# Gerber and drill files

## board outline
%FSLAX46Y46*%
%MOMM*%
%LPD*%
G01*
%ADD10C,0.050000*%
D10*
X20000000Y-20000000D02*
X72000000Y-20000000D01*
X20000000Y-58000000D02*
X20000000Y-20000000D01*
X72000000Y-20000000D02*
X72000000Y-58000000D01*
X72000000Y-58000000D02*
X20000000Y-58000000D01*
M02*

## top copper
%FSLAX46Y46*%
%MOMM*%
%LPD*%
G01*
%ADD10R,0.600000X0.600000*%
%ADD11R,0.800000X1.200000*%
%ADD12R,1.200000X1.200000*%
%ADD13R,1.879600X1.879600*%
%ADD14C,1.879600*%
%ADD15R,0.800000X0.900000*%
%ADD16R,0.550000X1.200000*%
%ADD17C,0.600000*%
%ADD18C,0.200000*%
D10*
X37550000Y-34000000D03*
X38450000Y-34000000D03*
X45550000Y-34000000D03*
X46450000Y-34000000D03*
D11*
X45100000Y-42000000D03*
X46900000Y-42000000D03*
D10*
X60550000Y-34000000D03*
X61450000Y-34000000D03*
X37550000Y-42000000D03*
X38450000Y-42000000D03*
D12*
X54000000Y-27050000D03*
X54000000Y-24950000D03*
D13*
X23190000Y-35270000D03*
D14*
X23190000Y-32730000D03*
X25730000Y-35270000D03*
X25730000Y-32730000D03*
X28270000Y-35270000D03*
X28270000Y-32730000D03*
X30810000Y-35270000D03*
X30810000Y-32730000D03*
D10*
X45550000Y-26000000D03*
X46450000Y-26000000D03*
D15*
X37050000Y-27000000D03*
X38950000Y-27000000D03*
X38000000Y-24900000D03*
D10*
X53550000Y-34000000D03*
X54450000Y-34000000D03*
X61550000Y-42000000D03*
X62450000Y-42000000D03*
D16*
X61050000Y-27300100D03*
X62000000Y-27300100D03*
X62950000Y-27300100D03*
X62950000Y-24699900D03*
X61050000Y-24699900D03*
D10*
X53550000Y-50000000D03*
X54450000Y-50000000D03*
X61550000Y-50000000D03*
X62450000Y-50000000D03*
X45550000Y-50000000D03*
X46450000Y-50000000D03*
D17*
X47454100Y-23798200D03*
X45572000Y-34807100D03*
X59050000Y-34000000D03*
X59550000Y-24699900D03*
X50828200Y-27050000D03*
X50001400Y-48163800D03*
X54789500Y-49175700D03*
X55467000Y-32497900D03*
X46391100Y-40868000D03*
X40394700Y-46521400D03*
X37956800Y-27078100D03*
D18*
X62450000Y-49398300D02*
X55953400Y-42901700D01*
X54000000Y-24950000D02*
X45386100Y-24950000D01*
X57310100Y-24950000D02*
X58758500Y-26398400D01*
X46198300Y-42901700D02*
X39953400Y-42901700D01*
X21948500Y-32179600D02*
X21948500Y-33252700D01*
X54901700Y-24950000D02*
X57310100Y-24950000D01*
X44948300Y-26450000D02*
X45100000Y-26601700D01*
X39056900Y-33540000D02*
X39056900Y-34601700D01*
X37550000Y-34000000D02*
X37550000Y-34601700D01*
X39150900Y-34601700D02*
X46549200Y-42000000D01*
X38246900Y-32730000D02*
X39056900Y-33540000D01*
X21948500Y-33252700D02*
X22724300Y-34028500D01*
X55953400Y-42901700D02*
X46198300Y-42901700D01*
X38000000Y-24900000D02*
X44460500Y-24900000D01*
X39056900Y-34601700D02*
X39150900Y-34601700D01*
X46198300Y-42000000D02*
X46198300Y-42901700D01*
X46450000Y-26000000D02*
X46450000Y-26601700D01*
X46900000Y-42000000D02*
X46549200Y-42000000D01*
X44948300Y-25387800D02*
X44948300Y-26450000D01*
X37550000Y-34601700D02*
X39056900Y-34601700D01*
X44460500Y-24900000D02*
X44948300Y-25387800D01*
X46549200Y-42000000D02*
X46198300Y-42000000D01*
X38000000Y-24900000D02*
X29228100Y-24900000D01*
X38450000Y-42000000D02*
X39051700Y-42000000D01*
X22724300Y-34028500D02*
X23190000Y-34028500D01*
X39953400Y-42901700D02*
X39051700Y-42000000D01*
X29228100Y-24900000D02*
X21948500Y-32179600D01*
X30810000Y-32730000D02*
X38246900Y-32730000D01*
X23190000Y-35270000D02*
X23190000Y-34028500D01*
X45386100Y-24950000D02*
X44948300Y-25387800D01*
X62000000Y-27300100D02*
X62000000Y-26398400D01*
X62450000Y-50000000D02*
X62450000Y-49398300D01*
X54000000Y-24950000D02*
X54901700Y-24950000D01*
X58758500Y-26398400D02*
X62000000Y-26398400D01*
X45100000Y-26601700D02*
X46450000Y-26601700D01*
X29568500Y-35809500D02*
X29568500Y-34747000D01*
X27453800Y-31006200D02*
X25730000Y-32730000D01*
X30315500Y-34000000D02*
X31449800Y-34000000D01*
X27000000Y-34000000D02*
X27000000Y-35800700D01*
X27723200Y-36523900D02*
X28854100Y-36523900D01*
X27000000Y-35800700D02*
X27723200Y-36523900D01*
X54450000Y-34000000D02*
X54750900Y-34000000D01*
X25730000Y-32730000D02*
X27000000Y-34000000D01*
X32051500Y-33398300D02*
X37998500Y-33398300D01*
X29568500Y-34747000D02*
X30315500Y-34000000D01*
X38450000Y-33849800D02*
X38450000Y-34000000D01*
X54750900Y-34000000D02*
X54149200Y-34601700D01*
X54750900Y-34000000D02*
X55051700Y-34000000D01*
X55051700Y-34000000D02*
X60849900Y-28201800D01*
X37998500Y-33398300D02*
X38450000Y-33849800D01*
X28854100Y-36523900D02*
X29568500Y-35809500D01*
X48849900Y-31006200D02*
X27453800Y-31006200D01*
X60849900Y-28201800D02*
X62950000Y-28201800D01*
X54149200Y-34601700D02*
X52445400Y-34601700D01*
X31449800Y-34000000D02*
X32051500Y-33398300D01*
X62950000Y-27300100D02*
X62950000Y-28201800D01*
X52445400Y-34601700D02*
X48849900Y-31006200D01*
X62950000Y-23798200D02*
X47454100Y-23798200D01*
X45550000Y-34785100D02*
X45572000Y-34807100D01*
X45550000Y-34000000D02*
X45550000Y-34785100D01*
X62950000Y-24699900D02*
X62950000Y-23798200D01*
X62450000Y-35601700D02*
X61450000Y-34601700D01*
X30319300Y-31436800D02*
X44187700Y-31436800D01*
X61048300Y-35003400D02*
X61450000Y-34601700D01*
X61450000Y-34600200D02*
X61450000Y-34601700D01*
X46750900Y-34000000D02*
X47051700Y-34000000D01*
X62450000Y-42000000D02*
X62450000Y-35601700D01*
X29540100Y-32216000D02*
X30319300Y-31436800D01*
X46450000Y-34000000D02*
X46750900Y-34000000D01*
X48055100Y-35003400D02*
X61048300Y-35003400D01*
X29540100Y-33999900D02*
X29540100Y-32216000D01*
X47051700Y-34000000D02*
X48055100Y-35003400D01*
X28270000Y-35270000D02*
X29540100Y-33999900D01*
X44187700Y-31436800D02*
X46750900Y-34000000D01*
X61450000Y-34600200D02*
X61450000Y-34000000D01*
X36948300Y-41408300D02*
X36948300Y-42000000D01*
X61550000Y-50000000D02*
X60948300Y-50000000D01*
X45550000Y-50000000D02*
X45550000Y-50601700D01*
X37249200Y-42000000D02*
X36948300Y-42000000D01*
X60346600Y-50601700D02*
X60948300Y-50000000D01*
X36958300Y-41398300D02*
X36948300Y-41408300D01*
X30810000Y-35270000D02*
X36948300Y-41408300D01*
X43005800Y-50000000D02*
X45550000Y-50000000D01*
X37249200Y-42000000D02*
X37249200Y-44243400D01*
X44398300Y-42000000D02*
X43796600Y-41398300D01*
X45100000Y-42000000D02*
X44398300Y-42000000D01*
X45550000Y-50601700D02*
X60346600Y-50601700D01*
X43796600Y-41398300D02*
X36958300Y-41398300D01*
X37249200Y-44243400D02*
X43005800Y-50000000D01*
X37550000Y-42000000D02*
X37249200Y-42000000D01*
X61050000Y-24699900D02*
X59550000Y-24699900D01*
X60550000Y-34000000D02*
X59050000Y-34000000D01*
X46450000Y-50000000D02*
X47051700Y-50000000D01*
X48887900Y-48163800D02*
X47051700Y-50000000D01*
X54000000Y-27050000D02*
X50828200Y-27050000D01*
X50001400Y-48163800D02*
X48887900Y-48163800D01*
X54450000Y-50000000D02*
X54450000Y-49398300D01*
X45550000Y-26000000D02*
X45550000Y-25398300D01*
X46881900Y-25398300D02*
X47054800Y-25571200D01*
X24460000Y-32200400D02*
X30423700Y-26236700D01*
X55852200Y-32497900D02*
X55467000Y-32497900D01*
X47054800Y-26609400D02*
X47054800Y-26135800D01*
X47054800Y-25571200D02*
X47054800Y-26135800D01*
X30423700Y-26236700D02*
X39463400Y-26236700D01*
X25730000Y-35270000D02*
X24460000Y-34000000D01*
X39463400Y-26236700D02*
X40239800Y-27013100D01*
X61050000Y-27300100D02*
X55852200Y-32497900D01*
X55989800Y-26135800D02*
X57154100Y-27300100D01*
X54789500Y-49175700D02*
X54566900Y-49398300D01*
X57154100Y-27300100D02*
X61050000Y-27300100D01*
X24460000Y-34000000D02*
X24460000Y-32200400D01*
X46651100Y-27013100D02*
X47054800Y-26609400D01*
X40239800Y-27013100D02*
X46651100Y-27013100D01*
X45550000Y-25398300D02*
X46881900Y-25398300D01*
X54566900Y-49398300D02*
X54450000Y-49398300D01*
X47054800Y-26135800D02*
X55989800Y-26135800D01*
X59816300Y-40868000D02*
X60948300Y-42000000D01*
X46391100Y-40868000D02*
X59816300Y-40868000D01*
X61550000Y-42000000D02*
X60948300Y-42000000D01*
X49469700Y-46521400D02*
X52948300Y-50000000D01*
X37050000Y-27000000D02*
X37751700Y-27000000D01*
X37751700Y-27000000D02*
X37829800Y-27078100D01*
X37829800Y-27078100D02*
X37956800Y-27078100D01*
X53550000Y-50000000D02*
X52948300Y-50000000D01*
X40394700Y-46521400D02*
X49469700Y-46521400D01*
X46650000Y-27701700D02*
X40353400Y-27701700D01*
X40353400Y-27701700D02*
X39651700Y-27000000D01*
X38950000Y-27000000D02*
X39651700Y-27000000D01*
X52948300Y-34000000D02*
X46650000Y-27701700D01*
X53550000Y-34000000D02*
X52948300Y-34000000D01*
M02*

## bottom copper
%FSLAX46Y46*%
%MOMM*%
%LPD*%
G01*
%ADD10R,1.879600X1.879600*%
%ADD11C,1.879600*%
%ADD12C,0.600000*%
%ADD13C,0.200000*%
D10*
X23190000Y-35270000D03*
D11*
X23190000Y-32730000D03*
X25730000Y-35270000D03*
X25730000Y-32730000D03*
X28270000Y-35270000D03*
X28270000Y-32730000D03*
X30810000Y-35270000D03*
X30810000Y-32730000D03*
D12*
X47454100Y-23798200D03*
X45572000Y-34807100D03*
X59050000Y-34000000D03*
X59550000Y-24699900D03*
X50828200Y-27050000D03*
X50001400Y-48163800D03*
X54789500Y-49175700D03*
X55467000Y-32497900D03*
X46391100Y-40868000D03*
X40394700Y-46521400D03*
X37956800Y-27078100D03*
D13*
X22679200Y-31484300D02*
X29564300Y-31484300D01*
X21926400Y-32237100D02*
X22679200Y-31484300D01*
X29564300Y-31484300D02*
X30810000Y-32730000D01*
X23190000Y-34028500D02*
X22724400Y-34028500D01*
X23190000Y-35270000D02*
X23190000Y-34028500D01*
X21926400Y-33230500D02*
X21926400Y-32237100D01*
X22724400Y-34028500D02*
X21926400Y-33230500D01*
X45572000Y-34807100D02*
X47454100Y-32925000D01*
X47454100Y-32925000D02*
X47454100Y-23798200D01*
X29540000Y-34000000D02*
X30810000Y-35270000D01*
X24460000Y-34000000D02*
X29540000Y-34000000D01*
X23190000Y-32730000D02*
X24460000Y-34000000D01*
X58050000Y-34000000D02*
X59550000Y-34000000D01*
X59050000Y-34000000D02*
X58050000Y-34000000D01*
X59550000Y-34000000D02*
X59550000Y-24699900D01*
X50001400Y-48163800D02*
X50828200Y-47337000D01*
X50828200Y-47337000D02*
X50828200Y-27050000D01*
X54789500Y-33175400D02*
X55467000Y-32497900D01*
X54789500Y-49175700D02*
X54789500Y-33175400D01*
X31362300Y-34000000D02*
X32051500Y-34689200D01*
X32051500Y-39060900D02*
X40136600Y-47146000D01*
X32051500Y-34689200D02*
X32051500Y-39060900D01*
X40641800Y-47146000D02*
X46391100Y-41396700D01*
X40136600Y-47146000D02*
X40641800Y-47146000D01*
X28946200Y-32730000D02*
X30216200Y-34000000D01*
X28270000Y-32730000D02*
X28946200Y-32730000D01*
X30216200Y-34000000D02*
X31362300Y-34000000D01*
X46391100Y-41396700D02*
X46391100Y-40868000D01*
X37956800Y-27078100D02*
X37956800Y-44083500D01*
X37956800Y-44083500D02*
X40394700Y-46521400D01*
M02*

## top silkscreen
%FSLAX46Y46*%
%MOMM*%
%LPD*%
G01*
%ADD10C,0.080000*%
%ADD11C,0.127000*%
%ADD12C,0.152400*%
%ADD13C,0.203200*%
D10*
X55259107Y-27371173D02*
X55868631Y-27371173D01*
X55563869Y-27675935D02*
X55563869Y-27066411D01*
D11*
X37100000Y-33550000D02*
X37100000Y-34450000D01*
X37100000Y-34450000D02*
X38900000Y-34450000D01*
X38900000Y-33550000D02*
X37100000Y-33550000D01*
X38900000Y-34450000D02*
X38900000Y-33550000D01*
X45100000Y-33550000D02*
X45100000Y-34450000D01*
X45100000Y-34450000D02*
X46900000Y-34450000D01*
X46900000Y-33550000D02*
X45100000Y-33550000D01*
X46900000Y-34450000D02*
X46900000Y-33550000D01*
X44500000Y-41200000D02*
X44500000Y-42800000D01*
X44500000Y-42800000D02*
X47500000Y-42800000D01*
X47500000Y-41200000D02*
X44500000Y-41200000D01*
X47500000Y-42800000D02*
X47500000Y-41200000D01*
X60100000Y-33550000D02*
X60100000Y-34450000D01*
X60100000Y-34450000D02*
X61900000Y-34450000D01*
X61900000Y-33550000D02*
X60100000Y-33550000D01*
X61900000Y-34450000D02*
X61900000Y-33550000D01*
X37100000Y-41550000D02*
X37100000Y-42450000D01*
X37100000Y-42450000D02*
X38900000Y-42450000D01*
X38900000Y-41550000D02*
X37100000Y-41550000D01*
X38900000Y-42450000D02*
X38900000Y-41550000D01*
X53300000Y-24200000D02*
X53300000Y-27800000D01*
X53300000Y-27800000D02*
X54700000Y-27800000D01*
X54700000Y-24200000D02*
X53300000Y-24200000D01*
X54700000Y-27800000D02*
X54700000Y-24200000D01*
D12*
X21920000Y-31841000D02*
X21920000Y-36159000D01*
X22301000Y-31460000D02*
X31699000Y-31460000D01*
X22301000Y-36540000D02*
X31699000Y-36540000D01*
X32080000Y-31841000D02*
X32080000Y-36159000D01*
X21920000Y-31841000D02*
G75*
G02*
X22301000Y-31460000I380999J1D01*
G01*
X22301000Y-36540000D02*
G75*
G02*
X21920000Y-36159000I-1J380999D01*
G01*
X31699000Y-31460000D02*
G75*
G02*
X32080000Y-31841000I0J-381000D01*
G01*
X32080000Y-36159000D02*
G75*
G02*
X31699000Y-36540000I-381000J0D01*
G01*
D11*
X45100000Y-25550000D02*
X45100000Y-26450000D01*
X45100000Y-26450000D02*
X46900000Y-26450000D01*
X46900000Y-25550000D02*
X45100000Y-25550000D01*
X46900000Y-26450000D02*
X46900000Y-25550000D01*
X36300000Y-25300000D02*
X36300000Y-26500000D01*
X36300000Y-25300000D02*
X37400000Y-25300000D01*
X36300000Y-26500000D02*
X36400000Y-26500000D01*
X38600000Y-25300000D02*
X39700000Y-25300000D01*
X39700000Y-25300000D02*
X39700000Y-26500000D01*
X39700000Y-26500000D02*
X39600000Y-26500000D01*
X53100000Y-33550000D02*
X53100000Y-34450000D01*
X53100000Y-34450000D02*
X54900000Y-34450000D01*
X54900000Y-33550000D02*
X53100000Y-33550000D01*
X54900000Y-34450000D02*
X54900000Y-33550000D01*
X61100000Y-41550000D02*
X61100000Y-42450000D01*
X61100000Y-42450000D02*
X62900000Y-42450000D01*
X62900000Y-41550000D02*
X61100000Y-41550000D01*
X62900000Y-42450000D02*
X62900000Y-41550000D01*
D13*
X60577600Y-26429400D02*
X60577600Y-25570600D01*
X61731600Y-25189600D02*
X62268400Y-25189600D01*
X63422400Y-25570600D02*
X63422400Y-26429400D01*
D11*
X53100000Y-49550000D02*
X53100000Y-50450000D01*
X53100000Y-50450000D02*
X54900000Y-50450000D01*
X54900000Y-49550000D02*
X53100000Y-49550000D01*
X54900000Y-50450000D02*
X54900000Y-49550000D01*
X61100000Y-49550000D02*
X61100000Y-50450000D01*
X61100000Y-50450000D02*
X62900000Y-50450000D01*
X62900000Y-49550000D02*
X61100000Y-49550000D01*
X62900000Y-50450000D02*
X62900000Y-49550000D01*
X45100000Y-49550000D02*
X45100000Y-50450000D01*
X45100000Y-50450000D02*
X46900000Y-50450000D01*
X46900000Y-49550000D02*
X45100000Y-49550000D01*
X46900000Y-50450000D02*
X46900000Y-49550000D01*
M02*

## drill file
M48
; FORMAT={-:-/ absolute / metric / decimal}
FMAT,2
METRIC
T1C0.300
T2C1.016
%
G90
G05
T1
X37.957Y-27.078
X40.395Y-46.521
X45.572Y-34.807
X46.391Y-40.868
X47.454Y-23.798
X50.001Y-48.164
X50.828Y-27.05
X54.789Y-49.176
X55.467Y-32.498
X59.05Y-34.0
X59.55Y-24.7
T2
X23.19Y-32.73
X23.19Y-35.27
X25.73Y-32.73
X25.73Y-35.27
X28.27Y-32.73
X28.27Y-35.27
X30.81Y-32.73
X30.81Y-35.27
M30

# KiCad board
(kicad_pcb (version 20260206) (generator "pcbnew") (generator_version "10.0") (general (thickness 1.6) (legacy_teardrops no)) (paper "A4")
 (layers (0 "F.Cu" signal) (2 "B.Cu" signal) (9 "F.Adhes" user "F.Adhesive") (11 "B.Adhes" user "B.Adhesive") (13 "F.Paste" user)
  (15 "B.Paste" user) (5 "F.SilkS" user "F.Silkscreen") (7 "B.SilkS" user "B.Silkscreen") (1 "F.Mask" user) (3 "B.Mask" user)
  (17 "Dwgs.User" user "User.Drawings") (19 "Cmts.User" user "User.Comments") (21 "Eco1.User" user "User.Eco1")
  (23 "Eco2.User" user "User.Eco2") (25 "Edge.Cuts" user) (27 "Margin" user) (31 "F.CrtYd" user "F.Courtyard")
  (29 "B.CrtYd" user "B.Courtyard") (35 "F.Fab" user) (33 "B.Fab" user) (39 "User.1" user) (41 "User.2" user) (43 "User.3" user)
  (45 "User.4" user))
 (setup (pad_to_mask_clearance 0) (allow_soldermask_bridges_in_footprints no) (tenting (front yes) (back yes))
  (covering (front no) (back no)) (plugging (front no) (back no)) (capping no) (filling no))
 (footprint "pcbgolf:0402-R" (layer "F.Cu") (at 38 34)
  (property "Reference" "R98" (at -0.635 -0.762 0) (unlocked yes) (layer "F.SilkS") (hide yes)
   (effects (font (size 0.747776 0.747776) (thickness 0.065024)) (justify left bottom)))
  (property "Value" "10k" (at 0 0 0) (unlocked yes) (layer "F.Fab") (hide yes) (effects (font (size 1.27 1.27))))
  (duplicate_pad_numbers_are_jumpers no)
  (fp_line (start -0.9 -0.45) (end -0.9 0.45) (stroke (width 0.127) (type solid)) (layer "F.SilkS"))
  (fp_line (start -0.9 0.45) (end 0.9 0.45) (stroke (width 0.127) (type solid)) (layer "F.SilkS"))
  (fp_line (start 0.9 -0.45) (end -0.9 -0.45) (stroke (width 0.127) (type solid)) (layer "F.SilkS"))
  (fp_line (start 0.9 0.45) (end 0.9 -0.45) (stroke (width 0.127) (type solid)) (layer "F.SilkS"))
  (pad "1" smd rect (at -0.45 0) (size 0.6 0.6) (layers "F.Cu" "F.Mask" "F.Paste") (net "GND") (solder_mask_margin 0.0508)
   (solder_paste_margin 0) (thermal_bridge_angle 0))
  (pad "2" smd rect (at 0.45 0) (size 0.6 0.6) (layers "F.Cu" "F.Mask" "F.Paste") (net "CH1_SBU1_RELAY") (solder_mask_margin 0.0508)
   (solder_paste_margin 0) (thermal_bridge_angle 0)))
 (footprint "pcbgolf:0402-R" (layer "F.Cu") (at 46 34)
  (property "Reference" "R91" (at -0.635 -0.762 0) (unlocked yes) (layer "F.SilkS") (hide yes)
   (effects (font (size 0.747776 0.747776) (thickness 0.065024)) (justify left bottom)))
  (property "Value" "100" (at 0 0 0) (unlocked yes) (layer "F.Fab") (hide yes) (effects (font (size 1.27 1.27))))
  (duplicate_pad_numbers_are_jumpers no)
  (fp_line (start -0.9 -0.45) (end -0.9 0.45) (stroke (width 0.127) (type solid)) (layer "F.SilkS"))
  (fp_line (start -0.9 0.45) (end 0.9 0.45) (stroke (width 0.127) (type solid)) (layer "F.SilkS"))
  (fp_line (start 0.9 -0.45) (end -0.9 -0.45) (stroke (width 0.127) (type solid)) (layer "F.SilkS"))
  (fp_line (start 0.9 0.45) (end 0.9 -0.45) (stroke (width 0.127) (type solid)) (layer "F.SilkS"))
  (pad "1" smd rect (at -0.45 0) (size 0.6 0.6) (layers "F.Cu" "F.Mask" "F.Paste") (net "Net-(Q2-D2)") (solder_mask_margin 0.0508)
   (solder_paste_margin 0) (thermal_bridge_angle 0))
  (pad "2" smd rect (at 0.45 0) (size 0.6 0.6) (layers "F.Cu" "F.Mask" "F.Paste") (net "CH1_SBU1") (solder_mask_margin 0.0508)
   (solder_paste_margin 0) (thermal_bridge_angle 0)))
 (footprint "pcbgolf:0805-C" (layer "F.Cu") (at 46 42)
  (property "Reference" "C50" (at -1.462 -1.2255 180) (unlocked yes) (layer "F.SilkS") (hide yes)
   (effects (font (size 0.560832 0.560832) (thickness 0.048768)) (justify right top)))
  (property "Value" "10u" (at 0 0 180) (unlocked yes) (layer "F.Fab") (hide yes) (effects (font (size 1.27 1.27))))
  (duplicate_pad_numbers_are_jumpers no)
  (fp_line (start -1.5 -0.8) (end -1.5 0.8) (stroke (width 0.127) (type solid)) (layer "F.SilkS"))
  (fp_line (start -1.5 0.8) (end 1.5 0.8) (stroke (width 0.127) (type solid)) (layer "F.SilkS"))
  (fp_line (start 1.5 -0.8) (end -1.5 -0.8) (stroke (width 0.127) (type solid)) (layer "F.SilkS"))
  (fp_line (start 1.5 0.8) (end 1.5 -0.8) (stroke (width 0.127) (type solid)) (layer "F.SilkS"))
  (pad "1" smd rect (at -0.9 0) (size 0.8 1.2) (layers "F.Cu" "F.Mask" "F.Paste") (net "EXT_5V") (solder_mask_margin 0.0508)
   (solder_paste_margin 0) (thermal_bridge_angle 0))
  (pad "2" smd rect (at 0.9 0) (size 0.8 1.2) (layers "F.Cu" "F.Mask" "F.Paste") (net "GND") (solder_mask_margin 0.0508)
   (solder_paste_margin 0) (thermal_bridge_angle 0)))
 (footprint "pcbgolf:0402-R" (layer "F.Cu") (at 61 34)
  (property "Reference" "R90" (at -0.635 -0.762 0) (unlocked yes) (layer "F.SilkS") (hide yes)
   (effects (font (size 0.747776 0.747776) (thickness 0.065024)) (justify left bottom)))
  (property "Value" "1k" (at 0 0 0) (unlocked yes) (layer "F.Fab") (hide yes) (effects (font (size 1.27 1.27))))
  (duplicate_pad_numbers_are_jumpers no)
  (fp_line (start -0.9 -0.45) (end -0.9 0.45) (stroke (width 0.127) (type solid)) (layer "F.SilkS"))
  (fp_line (start -0.9 0.45) (end 0.9 0.45) (stroke (width 0.127) (type solid)) (layer "F.SilkS"))
  (fp_line (start 0.9 -0.45) (end -0.9 -0.45) (stroke (width 0.127) (type solid)) (layer "F.SilkS"))
  (fp_line (start 0.9 0.45) (end 0.9 -0.45) (stroke (width 0.127) (type solid)) (layer "F.SilkS"))
  (pad "1" smd rect (at -0.45 0) (size 0.6 0.6) (layers "F.Cu" "F.Mask" "F.Paste") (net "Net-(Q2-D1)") (solder_mask_margin 0.0508)
   (solder_paste_margin 0) (thermal_bridge_angle 0))
  (pad "2" smd rect (at 0.45 0) (size 0.6 0.6) (layers "F.Cu" "F.Mask" "F.Paste") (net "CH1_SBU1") (solder_mask_margin 0.0508)
   (solder_paste_margin 0) (thermal_bridge_angle 0)))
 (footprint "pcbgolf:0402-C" (layer "F.Cu") (at 38 42)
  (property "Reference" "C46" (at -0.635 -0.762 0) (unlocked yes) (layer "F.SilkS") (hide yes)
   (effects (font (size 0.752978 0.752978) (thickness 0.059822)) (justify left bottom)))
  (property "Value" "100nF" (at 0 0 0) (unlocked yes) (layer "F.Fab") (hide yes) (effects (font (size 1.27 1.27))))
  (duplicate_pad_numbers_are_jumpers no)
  (fp_line (start -0.9 -0.45) (end -0.9 0.45) (stroke (width 0.127) (type solid)) (layer "F.SilkS"))
  (fp_line (start -0.9 0.45) (end 0.9 0.45) (stroke (width 0.127) (type solid)) (layer "F.SilkS"))
  (fp_line (start 0.9 -0.45) (end -0.9 -0.45) (stroke (width 0.127) (type solid)) (layer "F.SilkS"))
  (fp_line (start 0.9 0.45) (end 0.9 -0.45) (stroke (width 0.127) (type solid)) (layer "F.SilkS"))
  (pad "1" smd rect (at -0.45 0) (size 0.6 0.6) (layers "F.Cu" "F.Mask" "F.Paste") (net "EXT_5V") (solder_mask_margin 0.0508)
   (solder_paste_margin 0) (thermal_bridge_angle 0))
  (pad "2" smd rect (at 0.45 0) (size 0.6 0.6) (layers "F.Cu" "F.Mask" "F.Paste") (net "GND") (solder_mask_margin 0.0508)
   (solder_paste_margin 0) (thermal_bridge_angle 0)))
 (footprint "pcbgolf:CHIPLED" (layer "F.Cu") (at 54 26)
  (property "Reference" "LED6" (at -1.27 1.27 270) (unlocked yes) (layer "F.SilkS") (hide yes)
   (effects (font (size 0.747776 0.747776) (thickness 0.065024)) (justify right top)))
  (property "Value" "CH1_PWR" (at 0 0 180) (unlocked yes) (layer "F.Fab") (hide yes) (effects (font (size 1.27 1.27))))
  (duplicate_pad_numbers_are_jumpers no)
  (fp_line (start -0.7 -1.8) (end -0.7 1.8) (stroke (width 0.127) (type solid)) (layer "F.SilkS"))
  (fp_line (start -0.7 1.8) (end 0.7 1.8) (stroke (width 0.127) (type solid)) (layer "F.SilkS"))
  (fp_line (start 0.7 -1.8) (end -0.7 -1.8) (stroke (width 0.127) (type solid)) (layer "F.SilkS"))
  (fp_line (start 0.7 1.8) (end 0.7 -1.8) (stroke (width 0.127) (type solid)) (layer "F.SilkS"))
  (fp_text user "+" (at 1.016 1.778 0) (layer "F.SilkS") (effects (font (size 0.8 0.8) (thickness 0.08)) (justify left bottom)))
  (pad "A" smd rect (at 0 1.05) (size 1.2 1.2) (layers "F.Cu" "F.Mask" "F.Paste") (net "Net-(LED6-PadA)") (solder_mask_margin 0.0508)
   (solder_paste_margin 0) (thermal_bridge_angle 0))
  (pad "C" smd rect (at 0 -1.05) (size 1.2 1.2) (layers "F.Cu" "F.Mask" "F.Paste") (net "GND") (solder_mask_margin 0.0508)
   (solder_paste_margin 0) (thermal_bridge_angle 0)))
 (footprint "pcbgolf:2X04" (layer "F.Cu") (at 27 34)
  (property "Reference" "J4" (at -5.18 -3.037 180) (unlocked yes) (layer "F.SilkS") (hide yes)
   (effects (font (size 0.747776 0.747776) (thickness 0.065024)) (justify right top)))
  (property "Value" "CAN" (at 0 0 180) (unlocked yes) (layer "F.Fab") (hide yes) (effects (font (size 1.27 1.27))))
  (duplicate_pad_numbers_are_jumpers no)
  (fp_line (start -5.08 -2.159) (end -5.08 2.159) (stroke (width 0.1524) (type solid)) (layer "F.SilkS"))
  (fp_line (start -4.699 -2.54) (end 4.699 -2.54) (stroke (width 0.1524) (type solid)) (layer "F.SilkS"))
  (fp_line (start -4.699 2.54) (end 4.699 2.54) (stroke (width 0.1524) (type solid)) (layer "F.SilkS"))
  (fp_line (start 5.08 -2.159) (end 5.08 2.159) (stroke (width 0.1524) (type solid)) (layer "F.SilkS"))
  (fp_arc (start -5.08 -2.159) (mid -4.968408 -2.428408) (end -4.699 -2.54) (stroke (width 0.1524) (type solid)) (layer "F.SilkS"))
  (fp_arc (start -4.699 2.54) (mid -4.968408 2.428408) (end -5.08 2.159) (stroke (width 0.1524) (type solid)) (layer "F.SilkS"))
  (fp_arc (start 4.699 -2.54) (mid 4.968408 -2.428408) (end 5.08 -2.159) (stroke (width 0.1524) (type solid)) (layer "F.SilkS"))
  (fp_arc (start 5.08 2.159) (mid 4.968408 2.428408) (end 4.699 2.54) (stroke (width 0.1524) (type solid)) (layer "F.SilkS"))
  (pad "1" thru_hole rect (at -3.81 1.27 90) (size 1.8796 1.8796) (drill 1.016) (layers "*.Cu" "*.Mask") (remove_unused_layers no)
   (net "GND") (solder_mask_margin 0.0508) (thermal_bridge_angle 0))
  (pad "2" thru_hole circle (at -3.81 -1.27 90) (size 1.8796 1.8796) (drill 1.016) (layers "*.Cu" "*.Mask") (remove_unused_layers no)
   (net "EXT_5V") (solder_mask_margin 0.0508) (thermal_bridge_angle 0))
  (pad "3" thru_hole circle (at -1.27 1.27 90) (size 1.8796 1.8796) (drill 1.016) (layers "*.Cu" "*.Mask") (remove_unused_layers no)
   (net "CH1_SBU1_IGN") (solder_mask_margin 0.0508) (thermal_bridge_angle 0))
  (pad "4" thru_hole circle (at -1.27 -1.27 90) (size 1.8796 1.8796) (drill 1.016) (layers "*.Cu" "*.Mask") (remove_unused_layers no)
   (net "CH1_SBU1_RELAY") (solder_mask_margin 0.0508) (thermal_bridge_angle 0))
  (pad "5" thru_hole circle (at 1.27 1.27 90) (size 1.8796 1.8796) (drill 1.016) (layers "*.Cu" "*.Mask") (remove_unused_layers no)
   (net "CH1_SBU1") (solder_mask_margin 0.0508) (thermal_bridge_angle 0))
  (pad "6" thru_hole circle (at 1.27 -1.27 90) (size 1.8796 1.8796) (drill 1.016) (layers "*.Cu" "*.Mask") (remove_unused_layers no)
   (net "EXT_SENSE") (solder_mask_margin 0.0508) (thermal_bridge_angle 0))
  (pad "7" thru_hole circle (at 3.81 1.27 90) (size 1.8796 1.8796) (drill 1.016) (layers "*.Cu" "*.Mask") (remove_unused_layers no)
   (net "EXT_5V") (solder_mask_margin 0.0508) (thermal_bridge_angle 0))
  (pad "8" thru_hole circle (at 3.81 -1.27 90) (size 1.8796 1.8796) (drill 1.016) (layers "*.Cu" "*.Mask") (remove_unused_layers no)
   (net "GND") (solder_mask_margin 0.0508) (thermal_bridge_angle 0)))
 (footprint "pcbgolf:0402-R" (layer "F.Cu") (at 46 26)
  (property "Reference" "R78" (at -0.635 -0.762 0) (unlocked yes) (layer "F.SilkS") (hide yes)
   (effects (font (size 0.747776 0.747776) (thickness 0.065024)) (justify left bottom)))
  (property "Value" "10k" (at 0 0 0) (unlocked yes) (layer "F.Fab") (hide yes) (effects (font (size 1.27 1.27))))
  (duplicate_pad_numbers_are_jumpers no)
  (fp_line (start -0.9 -0.45) (end -0.9 0.45) (stroke (width 0.127) (type solid)) (layer "F.SilkS"))
  (fp_line (start -0.9 0.45) (end 0.9 0.45) (stroke (width 0.127) (type solid)) (layer "F.SilkS"))
  (fp_line (start 0.9 -0.45) (end -0.9 -0.45) (stroke (width 0.127) (type solid)) (layer "F.SilkS"))
  (fp_line (start 0.9 0.45) (end 0.9 -0.45) (stroke (width 0.127) (type solid)) (layer "F.SilkS"))
  (pad "1" smd rect (at -0.45 0) (size 0.6 0.6) (layers "F.Cu" "F.Mask" "F.Paste") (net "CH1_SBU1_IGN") (solder_mask_margin 0.0508)
   (solder_paste_margin 0) (thermal_bridge_angle 0))
  (pad "2" smd rect (at 0.45 0) (size 0.6 0.6) (layers "F.Cu" "F.Mask" "F.Paste") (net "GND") (solder_mask_margin 0.0508)
   (solder_paste_margin 0) (thermal_bridge_angle 0)))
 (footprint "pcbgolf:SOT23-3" (layer "F.Cu") (at 38 26)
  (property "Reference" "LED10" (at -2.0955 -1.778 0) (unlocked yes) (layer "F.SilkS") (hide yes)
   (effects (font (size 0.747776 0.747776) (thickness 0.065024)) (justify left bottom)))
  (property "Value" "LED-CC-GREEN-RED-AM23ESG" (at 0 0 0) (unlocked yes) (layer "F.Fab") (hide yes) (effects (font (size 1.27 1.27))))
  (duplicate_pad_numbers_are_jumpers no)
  (fp_line (start -1.7 -0.7) (end -1.7 0.5) (stroke (width 0.127) (type solid)) (layer "F.SilkS"))
  (fp_line (start -1.7 -0.7) (end -0.6 -0.7) (stroke (width 0.127) (type solid)) (layer "F.SilkS"))
  (fp_line (start -1.7 0.5) (end -1.6 0.5) (stroke (width 0.127) (type solid)) (layer "F.SilkS"))
  (fp_line (start 0.6 -0.7) (end 1.7 -0.7) (stroke (width 0.127) (type solid)) (layer "F.SilkS"))
  (fp_line (start 1.7 -0.7) (end 1.7 0.5) (stroke (width 0.127) (type solid)) (layer "F.SilkS"))
  (fp_line (start 1.7 0.5) (end 1.6 0.5) (stroke (width 0.127) (type solid)) (layer "F.SilkS"))
  (pad "1" smd rect (at -0.95 1) (size 0.8 0.9) (layers "F.Cu" "F.Mask" "F.Paste") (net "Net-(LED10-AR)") (solder_mask_margin 0.0508)
   (solder_paste_margin 0) (thermal_bridge_angle 0))
  (pad "2" smd rect (at 0.95 1) (size 0.8 0.9) (layers "F.Cu" "F.Mask" "F.Paste") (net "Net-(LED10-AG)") (solder_mask_margin 0.0508)
   (solder_paste_margin 0) (thermal_bridge_angle 0))
  (pad "3" smd rect (at 0 -1.1) (size 0.8 0.9) (layers "F.Cu" "F.Mask" "F.Paste") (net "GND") (solder_mask_margin 0.0508)
   (solder_paste_margin 0) (thermal_bridge_angle 0)))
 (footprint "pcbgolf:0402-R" (layer "F.Cu") (at 54 34)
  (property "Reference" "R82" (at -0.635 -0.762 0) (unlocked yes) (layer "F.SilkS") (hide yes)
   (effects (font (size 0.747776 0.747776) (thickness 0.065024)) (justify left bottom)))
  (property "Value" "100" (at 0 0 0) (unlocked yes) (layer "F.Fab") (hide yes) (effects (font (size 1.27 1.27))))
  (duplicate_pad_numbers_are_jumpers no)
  (fp_line (start -0.9 -0.45) (end -0.9 0.45) (stroke (width 0.127) (type solid)) (layer "F.SilkS"))
  (fp_line (start -0.9 0.45) (end 0.9 0.45) (stroke (width 0.127) (type solid)) (layer "F.SilkS"))
  (fp_line (start 0.9 -0.45) (end -0.9 -0.45) (stroke (width 0.127) (type solid)) (layer "F.SilkS"))
  (fp_line (start 0.9 0.45) (end 0.9 -0.45) (stroke (width 0.127) (type solid)) (layer "F.SilkS"))
  (pad "1" smd rect (at -0.45 0) (size 0.6 0.6) (layers "F.Cu" "F.Mask" "F.Paste") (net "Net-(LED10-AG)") (solder_mask_margin 0.0508)
   (solder_paste_margin 0) (thermal_bridge_angle 0))
  (pad "2" smd rect (at 0.45 0) (size 0.6 0.6) (layers "F.Cu" "F.Mask" "F.Paste") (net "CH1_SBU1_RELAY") (solder_mask_margin 0.0508)
   (solder_paste_margin 0) (thermal_bridge_angle 0)))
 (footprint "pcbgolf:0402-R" (layer "F.Cu") (at 62 42)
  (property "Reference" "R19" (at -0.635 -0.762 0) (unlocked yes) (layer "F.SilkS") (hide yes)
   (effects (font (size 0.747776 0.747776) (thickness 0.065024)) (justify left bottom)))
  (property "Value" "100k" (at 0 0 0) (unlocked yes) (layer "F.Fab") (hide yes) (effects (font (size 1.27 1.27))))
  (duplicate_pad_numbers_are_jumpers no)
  (fp_line (start -0.9 -0.45) (end -0.9 0.45) (stroke (width 0.127) (type solid)) (layer "F.SilkS"))
  (fp_line (start -0.9 0.45) (end 0.9 0.45) (stroke (width 0.127) (type solid)) (layer "F.SilkS"))
  (fp_line (start 0.9 -0.45) (end -0.9 -0.45) (stroke (width 0.127) (type solid)) (layer "F.SilkS"))
  (fp_line (start 0.9 0.45) (end 0.9 -0.45) (stroke (width 0.127) (type solid)) (layer "F.SilkS"))
  (pad "1" smd rect (at -0.45 0) (size 0.6 0.6) (layers "F.Cu" "F.Mask" "F.Paste") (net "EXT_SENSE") (solder_mask_margin 0.0508)
   (solder_paste_margin 0) (thermal_bridge_angle 0))
  (pad "2" smd rect (at 0.45 0) (size 0.6 0.6) (layers "F.Cu" "F.Mask" "F.Paste") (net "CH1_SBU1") (solder_mask_margin 0.0508)
   (solder_paste_margin 0) (thermal_bridge_angle 0)))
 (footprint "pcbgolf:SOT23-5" (layer "F.Cu") (at 62 26)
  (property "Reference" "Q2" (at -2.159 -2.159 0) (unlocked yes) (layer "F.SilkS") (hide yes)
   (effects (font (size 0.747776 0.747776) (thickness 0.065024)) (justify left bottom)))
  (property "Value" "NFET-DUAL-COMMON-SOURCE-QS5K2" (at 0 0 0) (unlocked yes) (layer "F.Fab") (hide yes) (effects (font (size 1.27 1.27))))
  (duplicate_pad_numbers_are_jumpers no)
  (fp_line (start -1.4224 0.4294) (end -1.4224 -0.4294) (stroke (width 0.2032) (type solid)) (layer "F.SilkS"))
  (fp_line (start -0.2684 -0.8104) (end 0.2684 -0.8104) (stroke (width 0.2032) (type solid)) (layer "F.SilkS"))
  (fp_line (start 1.4224 -0.4294) (end 1.4224 0.4294) (stroke (width 0.2032) (type solid)) (layer "F.SilkS"))
  (pad "1" smd rect (at -0.95 1.3001) (size 0.55 1.2) (layers "F.Cu" "F.Mask" "F.Paste") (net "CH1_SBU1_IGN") (solder_mask_margin 0.0508)
   (solder_paste_margin 0) (thermal_bridge_angle 0))
  (pad "2" smd rect (at 0 1.3001) (size 0.55 1.2) (layers "F.Cu" "F.Mask" "F.Paste") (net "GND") (solder_mask_margin 0.0508)
   (solder_paste_margin 0) (thermal_bridge_angle 0))
  (pad "3" smd rect (at 0.95 1.3001) (size 0.55 1.2) (layers "F.Cu" "F.Mask" "F.Paste") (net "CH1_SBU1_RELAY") (solder_mask_margin 0.0508)
   (solder_paste_margin 0) (thermal_bridge_angle 0))
  (pad "4" smd rect (at 0.95 -1.3001) (size 0.55 1.2) (layers "F.Cu" "F.Mask" "F.Paste") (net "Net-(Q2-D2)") (solder_mask_margin 0.0508)
   (solder_paste_margin 0) (thermal_bridge_angle 0))
  (pad "5" smd rect (at -0.95 -1.3001) (size 0.55 1.2) (layers "F.Cu" "F.Mask" "F.Paste") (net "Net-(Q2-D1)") (solder_mask_margin 0.0508)
   (solder_paste_margin 0) (thermal_bridge_angle 0)))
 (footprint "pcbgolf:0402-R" (layer "F.Cu") (at 54 50)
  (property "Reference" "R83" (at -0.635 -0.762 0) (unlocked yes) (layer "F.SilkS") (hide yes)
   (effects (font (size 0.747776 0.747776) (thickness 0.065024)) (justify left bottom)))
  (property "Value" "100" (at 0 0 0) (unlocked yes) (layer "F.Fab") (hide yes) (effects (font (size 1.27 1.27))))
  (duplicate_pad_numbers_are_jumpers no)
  (fp_line (start -0.9 -0.45) (end -0.9 0.45) (stroke (width 0.127) (type solid)) (layer "F.SilkS"))
  (fp_line (start -0.9 0.45) (end 0.9 0.45) (stroke (width 0.127) (type solid)) (layer "F.SilkS"))
  (fp_line (start 0.9 -0.45) (end -0.9 -0.45) (stroke (width 0.127) (type solid)) (layer "F.SilkS"))
  (fp_line (start 0.9 0.45) (end 0.9 -0.45) (stroke (width 0.127) (type solid)) (layer "F.SilkS"))
  (pad "1" smd rect (at -0.45 0) (size 0.6 0.6) (layers "F.Cu" "F.Mask" "F.Paste") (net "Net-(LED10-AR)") (solder_mask_margin 0.0508)
   (solder_paste_margin 0) (thermal_bridge_angle 0))
  (pad "2" smd rect (at 0.45 0) (size 0.6 0.6) (layers "F.Cu" "F.Mask" "F.Paste") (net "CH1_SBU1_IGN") (solder_mask_margin 0.0508)
   (solder_paste_margin 0) (thermal_bridge_angle 0)))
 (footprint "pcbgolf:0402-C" (layer "F.Cu") (at 62 50)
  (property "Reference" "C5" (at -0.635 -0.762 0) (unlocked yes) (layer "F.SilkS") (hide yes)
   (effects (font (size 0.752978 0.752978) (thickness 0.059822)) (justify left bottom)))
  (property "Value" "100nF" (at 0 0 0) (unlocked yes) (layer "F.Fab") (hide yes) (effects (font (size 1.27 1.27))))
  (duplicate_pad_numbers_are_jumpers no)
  (fp_line (start -0.9 -0.45) (end -0.9 0.45) (stroke (width 0.127) (type solid)) (layer "F.SilkS"))
  (fp_line (start -0.9 0.45) (end 0.9 0.45) (stroke (width 0.127) (type solid)) (layer "F.SilkS"))
  (fp_line (start 0.9 -0.45) (end -0.9 -0.45) (stroke (width 0.127) (type solid)) (layer "F.SilkS"))
  (fp_line (start 0.9 0.45) (end 0.9 -0.45) (stroke (width 0.127) (type solid)) (layer "F.SilkS"))
  (pad "1" smd rect (at -0.45 0) (size 0.6 0.6) (layers "F.Cu" "F.Mask" "F.Paste") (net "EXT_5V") (solder_mask_margin 0.0508)
   (solder_paste_margin 0) (thermal_bridge_angle 0))
  (pad "2" smd rect (at 0.45 0) (size 0.6 0.6) (layers "F.Cu" "F.Mask" "F.Paste") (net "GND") (solder_mask_margin 0.0508)
   (solder_paste_margin 0) (thermal_bridge_angle 0)))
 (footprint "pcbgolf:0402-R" (layer "F.Cu") (at 46 50)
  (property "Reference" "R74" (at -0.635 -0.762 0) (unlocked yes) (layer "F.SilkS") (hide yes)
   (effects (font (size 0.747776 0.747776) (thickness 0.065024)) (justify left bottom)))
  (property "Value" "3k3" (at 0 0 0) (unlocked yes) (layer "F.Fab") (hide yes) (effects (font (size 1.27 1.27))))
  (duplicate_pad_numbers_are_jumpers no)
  (fp_line (start -0.9 -0.45) (end -0.9 0.45) (stroke (width 0.127) (type solid)) (layer "F.SilkS"))
  (fp_line (start -0.9 0.45) (end 0.9 0.45) (stroke (width 0.127) (type solid)) (layer "F.SilkS"))
  (fp_line (start 0.9 -0.45) (end -0.9 -0.45) (stroke (width 0.127) (type solid)) (layer "F.SilkS"))
  (fp_line (start 0.9 0.45) (end 0.9 -0.45) (stroke (width 0.127) (type solid)) (layer "F.SilkS"))
  (pad "1" smd rect (at -0.45 0) (size 0.6 0.6) (layers "F.Cu" "F.Mask" "F.Paste") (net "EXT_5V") (solder_mask_margin 0.0508)
   (solder_paste_margin 0) (thermal_bridge_angle 0))
  (pad "2" smd rect (at 0.45 0) (size 0.6 0.6) (layers "F.Cu" "F.Mask" "F.Paste") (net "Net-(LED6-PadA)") (solder_mask_margin 0.0508)
   (solder_paste_margin 0) (thermal_bridge_angle 0)))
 (gr_line (start 20 20) (end 72 20) (stroke (width 0.05) (type default)) (layer "Edge.Cuts"))
 (gr_line (start 20 58) (end 20 20) (stroke (width 0.05) (type default)) (layer "Edge.Cuts"))
 (gr_line (start 72 20) (end 72 58) (stroke (width 0.05) (type default)) (layer "Edge.Cuts"))
 (gr_line (start 72 58) (end 20 58) (stroke (width 0.05) (type default)) (layer "Edge.Cuts"))
 (segment (start 62.45 49.3983) (end 55.9534 42.9017) (width 0.2) (layer "F.Cu") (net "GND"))
 (segment (start 54 24.95) (end 45.3861 24.95) (width 0.2) (layer "F.Cu") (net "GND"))
 (segment (start 57.3101 24.95) (end 58.7585 26.3984) (width 0.2) (layer "F.Cu") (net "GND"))
 (segment (start 46.1983 42.9017) (end 39.9534 42.9017) (width 0.2) (layer "F.Cu") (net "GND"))
 (segment (start 21.9485 32.1796) (end 21.9485 33.2527) (width 0.2) (layer "F.Cu") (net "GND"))
 (segment (start 54.9017 24.95) (end 57.3101 24.95) (width 0.2) (layer "F.Cu") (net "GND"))
 (segment (start 44.9483 26.45) (end 45.1 26.6017) (width 0.2) (layer "F.Cu") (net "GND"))
 (segment (start 39.0569 33.54) (end 39.0569 34.6017) (width 0.2) (layer "F.Cu") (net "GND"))
 (segment (start 37.55 34) (end 37.55 34.6017) (width 0.2) (layer "F.Cu") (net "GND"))
 (segment (start 39.1509 34.6017) (end 46.5492 42) (width 0.2) (layer "F.Cu") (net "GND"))
 (segment (start 38.2469 32.73) (end 39.0569 33.54) (width 0.2) (layer "F.Cu") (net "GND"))
 (segment (start 21.9485 33.2527) (end 22.7243 34.0285) (width 0.2) (layer "F.Cu") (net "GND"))
 (segment (start 55.9534 42.9017) (end 46.1983 42.9017) (width 0.2) (layer "F.Cu") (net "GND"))
 (segment (start 38 24.9) (end 44.4605 24.9) (width 0.2) (layer "F.Cu") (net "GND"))
 (segment (start 39.0569 34.6017) (end 39.1509 34.6017) (width 0.2) (layer "F.Cu") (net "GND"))
 (segment (start 46.1983 42) (end 46.1983 42.9017) (width 0.2) (layer "F.Cu") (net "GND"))
 (segment (start 46.45 26) (end 46.45 26.6017) (width 0.2) (layer "F.Cu") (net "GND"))
 (segment (start 46.9 42) (end 46.5492 42) (width 0.2) (layer "F.Cu") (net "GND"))
 (segment (start 44.9483 25.3878) (end 44.9483 26.45) (width 0.2) (layer "F.Cu") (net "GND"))
 (segment (start 37.55 34.6017) (end 39.0569 34.6017) (width 0.2) (layer "F.Cu") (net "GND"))
 (segment (start 44.4605 24.9) (end 44.9483 25.3878) (width 0.2) (layer "F.Cu") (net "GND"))
 (segment (start 46.5492 42) (end 46.1983 42) (width 0.2) (layer "F.Cu") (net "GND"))
 (segment (start 38 24.9) (end 29.2281 24.9) (width 0.2) (layer "F.Cu") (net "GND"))
 (segment (start 38.45 42) (end 39.0517 42) (width 0.2) (layer "F.Cu") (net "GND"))
 (segment (start 22.7243 34.0285) (end 23.19 34.0285) (width 0.2) (layer "F.Cu") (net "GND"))
 (segment (start 39.9534 42.9017) (end 39.0517 42) (width 0.2) (layer "F.Cu") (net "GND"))
 (segment (start 29.2281 24.9) (end 21.9485 32.1796) (width 0.2) (layer "F.Cu") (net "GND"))
 (segment (start 30.81 32.73) (end 38.2469 32.73) (width 0.2) (layer "F.Cu") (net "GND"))
 (segment (start 23.19 35.27) (end 23.19 34.0285) (width 0.2) (layer "F.Cu") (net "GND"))
 (segment (start 45.3861 24.95) (end 44.9483 25.3878) (width 0.2) (layer "F.Cu") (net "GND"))
 (segment (start 62 27.3001) (end 62 26.3984) (width 0.2) (layer "F.Cu") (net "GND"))
 (segment (start 62.45 50) (end 62.45 49.3983) (width 0.2) (layer "F.Cu") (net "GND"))
 (segment (start 54 24.95) (end 54.9017 24.95) (width 0.2) (layer "F.Cu") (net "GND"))
 (segment (start 58.7585 26.3984) (end 62 26.3984) (width 0.2) (layer "F.Cu") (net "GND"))
 (segment (start 45.1 26.6017) (end 46.45 26.6017) (width 0.2) (layer "F.Cu") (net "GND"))
 (segment (start 22.6792 31.4843) (end 29.5643 31.4843) (width 0.2) (layer "B.Cu") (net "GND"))
 (segment (start 21.9264 32.2371) (end 22.6792 31.4843) (width 0.2) (layer "B.Cu") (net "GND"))
 (segment (start 29.5643 31.4843) (end 30.81 32.73) (width 0.2) (layer "B.Cu") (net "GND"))
 (segment (start 23.19 34.0285) (end 22.7244 34.0285) (width 0.2) (layer "B.Cu") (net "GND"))
 (segment (start 23.19 35.27) (end 23.19 34.0285) (width 0.2) (layer "B.Cu") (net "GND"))
 (segment (start 21.9264 33.2305) (end 21.9264 32.2371) (width 0.2) (layer "B.Cu") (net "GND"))
 (segment (start 22.7244 34.0285) (end 21.9264 33.2305) (width 0.2) (layer "B.Cu") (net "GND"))
 (segment (start 29.5685 35.8095) (end 29.5685 34.747) (width 0.2) (layer "F.Cu") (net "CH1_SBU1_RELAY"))
 (segment (start 27.4538 31.0062) (end 25.73 32.73) (width 0.2) (layer "F.Cu") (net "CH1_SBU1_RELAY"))
 (segment (start 30.3155 34) (end 31.4498 34) (width 0.2) (layer "F.Cu") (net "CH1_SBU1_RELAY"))
 (segment (start 27 34) (end 27 35.8007) (width 0.2) (layer "F.Cu") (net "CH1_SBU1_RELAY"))
 (segment (start 27.7232 36.5239) (end 28.8541 36.5239) (width 0.2) (layer "F.Cu") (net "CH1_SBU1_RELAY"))
 (segment (start 27 35.8007) (end 27.7232 36.5239) (width 0.2) (layer "F.Cu") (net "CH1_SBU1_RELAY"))
 (segment (start 54.45 34) (end 54.7509 34) (width 0.2) (layer "F.Cu") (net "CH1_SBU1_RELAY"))
 (segment (start 25.73 32.73) (end 27 34) (width 0.2) (layer "F.Cu") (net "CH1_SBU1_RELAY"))
 (segment (start 32.0515 33.3983) (end 37.9985 33.3983) (width 0.2) (layer "F.Cu") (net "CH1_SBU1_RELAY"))
 (segment (start 29.5685 34.747) (end 30.3155 34) (width 0.2) (layer "F.Cu") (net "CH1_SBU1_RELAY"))
 (segment (start 38.45 33.8498) (end 38.45 34) (width 0.2) (layer "F.Cu") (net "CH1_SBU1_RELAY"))
 (segment (start 54.7509 34) (end 54.1492 34.6017) (width 0.2) (layer "F.Cu") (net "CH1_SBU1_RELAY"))
 (segment (start 54.7509 34) (end 55.0517 34) (width 0.2) (layer "F.Cu") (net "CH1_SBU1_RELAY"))
 (segment (start 55.0517 34) (end 60.8499 28.2018) (width 0.2) (layer "F.Cu") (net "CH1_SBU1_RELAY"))
 (segment (start 37.9985 33.3983) (end 38.45 33.8498) (width 0.2) (layer "F.Cu") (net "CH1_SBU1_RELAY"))
 (segment (start 28.8541 36.5239) (end 29.5685 35.8095) (width 0.2) (layer "F.Cu") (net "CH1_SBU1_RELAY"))
 (segment (start 48.8499 31.0062) (end 27.4538 31.0062) (width 0.2) (layer "F.Cu") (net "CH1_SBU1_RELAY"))
 (segment (start 60.8499 28.2018) (end 62.95 28.2018) (width 0.2) (layer "F.Cu") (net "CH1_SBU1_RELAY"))
 (segment (start 54.1492 34.6017) (end 52.4454 34.6017) (width 0.2) (layer "F.Cu") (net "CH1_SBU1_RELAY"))
 (segment (start 31.4498 34) (end 32.0515 33.3983) (width 0.2) (layer "F.Cu") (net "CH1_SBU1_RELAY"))
 (segment (start 62.95 27.3001) (end 62.95 28.2018) (width 0.2) (layer "F.Cu") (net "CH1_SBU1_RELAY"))
 (segment (start 52.4454 34.6017) (end 48.8499 31.0062) (width 0.2) (layer "F.Cu") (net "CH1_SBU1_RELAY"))
 (segment (start 62.95 23.7982) (end 47.4541 23.7982) (width 0.2) (layer "F.Cu") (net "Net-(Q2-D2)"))
 (segment (start 45.55 34.7851) (end 45.572 34.8071) (width 0.2) (layer "F.Cu") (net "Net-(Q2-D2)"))
 (segment (start 45.55 34) (end 45.55 34.7851) (width 0.2) (layer "F.Cu") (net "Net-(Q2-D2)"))
 (segment (start 62.95 24.6999) (end 62.95 23.7982) (width 0.2) (layer "F.Cu") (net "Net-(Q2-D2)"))
 (via (at 47.4541 23.7982) (size 0.6) (drill 0.3) (layers "F.Cu" "B.Cu") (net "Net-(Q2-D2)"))
 (via (at 45.572 34.8071) (size 0.6) (drill 0.3) (layers "F.Cu" "B.Cu") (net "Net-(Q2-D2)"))
 (segment (start 45.572 34.8071) (end 47.4541 32.925) (width 0.2) (layer "B.Cu") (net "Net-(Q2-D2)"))
 (segment (start 47.4541 32.925) (end 47.4541 23.7982) (width 0.2) (layer "B.Cu") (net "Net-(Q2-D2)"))
 (segment (start 62.45 35.6017) (end 61.45 34.6017) (width 0.2) (layer "F.Cu") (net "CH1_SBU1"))
 (segment (start 30.3193 31.4368) (end 44.1877 31.4368) (width 0.2) (layer "F.Cu") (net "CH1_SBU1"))
 (segment (start 61.0483 35.0034) (end 61.45 34.6017) (width 0.2) (layer "F.Cu") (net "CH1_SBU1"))
 (segment (start 61.45 34.6002) (end 61.45 34.6017) (width 0.2) (layer "F.Cu") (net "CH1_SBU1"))
 (segment (start 46.7509 34) (end 47.0517 34) (width 0.2) (layer "F.Cu") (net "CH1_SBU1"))
 (segment (start 62.45 42) (end 62.45 35.6017) (width 0.2) (layer "F.Cu") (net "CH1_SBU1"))
 (segment (start 29.5401 32.216) (end 30.3193 31.4368) (width 0.2) (layer "F.Cu") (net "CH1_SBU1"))
 (segment (start 46.45 34) (end 46.7509 34) (width 0.2) (layer "F.Cu") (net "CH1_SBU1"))
 (segment (start 48.0551 35.0034) (end 61.0483 35.0034) (width 0.2) (layer "F.Cu") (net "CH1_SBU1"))
 (segment (start 29.5401 33.9999) (end 29.5401 32.216) (width 0.2) (layer "F.Cu") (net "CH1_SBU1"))
 (segment (start 47.0517 34) (end 48.0551 35.0034) (width 0.2) (layer "F.Cu") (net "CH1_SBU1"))
 (segment (start 28.27 35.27) (end 29.5401 33.9999) (width 0.2) (layer "F.Cu") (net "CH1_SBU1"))
 (segment (start 44.1877 31.4368) (end 46.7509 34) (width 0.2) (layer "F.Cu") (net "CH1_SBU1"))
 (segment (start 61.45 34.6002) (end 61.45 34) (width 0.2) (layer "F.Cu") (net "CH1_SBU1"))
 (segment (start 36.9483 41.4083) (end 36.9483 42) (width 0.2) (layer "F.Cu") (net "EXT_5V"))
 (segment (start 61.55 50) (end 60.9483 50) (width 0.2) (layer "F.Cu") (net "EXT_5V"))
 (segment (start 45.55 50) (end 45.55 50.6017) (width 0.2) (layer "F.Cu") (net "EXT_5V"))
 (segment (start 37.2492 42) (end 36.9483 42) (width 0.2) (layer "F.Cu") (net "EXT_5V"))
 (segment (start 60.3466 50.6017) (end 60.9483 50) (width 0.2) (layer "F.Cu") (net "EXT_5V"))
 (segment (start 36.9583 41.3983) (end 36.9483 41.4083) (width 0.2) (layer "F.Cu") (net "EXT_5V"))
 (segment (start 30.81 35.27) (end 36.9483 41.4083) (width 0.2) (layer "F.Cu") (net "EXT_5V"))
 (segment (start 43.0058 50) (end 45.55 50) (width 0.2) (layer "F.Cu") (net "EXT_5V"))
 (segment (start 37.2492 42) (end 37.2492 44.2434) (width 0.2) (layer "F.Cu") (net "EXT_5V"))
 (segment (start 44.3983 42) (end 43.7966 41.3983) (width 0.2) (layer "F.Cu") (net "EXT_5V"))
 (segment (start 45.1 42) (end 44.3983 42) (width 0.2) (layer "F.Cu") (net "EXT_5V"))
 (segment (start 45.55 50.6017) (end 60.3466 50.6017) (width 0.2) (layer "F.Cu") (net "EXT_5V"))
 (segment (start 43.7966 41.3983) (end 36.9583 41.3983) (width 0.2) (layer "F.Cu") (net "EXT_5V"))
 (segment (start 37.2492 44.2434) (end 43.0058 50) (width 0.2) (layer "F.Cu") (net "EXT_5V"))
 (segment (start 37.55 42) (end 37.2492 42) (width 0.2) (layer "F.Cu") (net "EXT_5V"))
 (segment (start 29.54 34) (end 30.81 35.27) (width 0.2) (layer "B.Cu") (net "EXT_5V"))
 (segment (start 24.46 34) (end 29.54 34) (width 0.2) (layer "B.Cu") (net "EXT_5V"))
 (segment (start 23.19 32.73) (end 24.46 34) (width 0.2) (layer "B.Cu") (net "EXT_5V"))
 (segment (start 61.05 24.6999) (end 59.55 24.6999) (width 0.2) (layer "F.Cu") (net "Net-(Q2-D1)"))
 (segment (start 60.55 34) (end 59.05 34) (width 0.2) (layer "F.Cu") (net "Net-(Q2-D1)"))
 (via (at 59.05 34) (size 0.6) (drill 0.3) (layers "F.Cu" "B.Cu") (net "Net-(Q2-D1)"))
 (via (at 59.55 24.6999) (size 0.6) (drill 0.3) (layers "F.Cu" "B.Cu") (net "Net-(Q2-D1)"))
 (segment (start 58.05 34) (end 59.55 34) (width 0.2) (layer "B.Cu") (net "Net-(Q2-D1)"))
 (segment (start 59.05 34) (end 58.05 34) (width 0.2) (layer "B.Cu") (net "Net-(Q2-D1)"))
 (segment (start 59.55 34) (end 59.55 24.6999) (width 0.2) (layer "B.Cu") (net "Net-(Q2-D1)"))
 (segment (start 46.45 50) (end 47.0517 50) (width 0.2) (layer "F.Cu") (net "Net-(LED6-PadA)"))
 (segment (start 48.8879 48.1638) (end 47.0517 50) (width 0.2) (layer "F.Cu") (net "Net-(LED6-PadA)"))
 (segment (start 54 27.05) (end 50.8282 27.05) (width 0.2) (layer "F.Cu") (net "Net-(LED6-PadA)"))
 (segment (start 50.0014 48.1638) (end 48.8879 48.1638) (width 0.2) (layer "F.Cu") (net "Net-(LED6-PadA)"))
 (via (at 50.8282 27.05) (size 0.6) (drill 0.3) (layers "F.Cu" "B.Cu") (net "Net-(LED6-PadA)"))
 (via (at 50.0014 48.1638) (size 0.6) (drill 0.3) (layers "F.Cu" "B.Cu") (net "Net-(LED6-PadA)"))
 (segment (start 50.0014 48.1638) (end 50.8282 47.337) (width 0.2) (layer "B.Cu") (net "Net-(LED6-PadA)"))
 (segment (start 50.8282 47.337) (end 50.8282 27.05) (width 0.2) (layer "B.Cu") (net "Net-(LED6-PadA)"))
 (segment (start 54.45 50) (end 54.45 49.3983) (width 0.2) (layer "F.Cu") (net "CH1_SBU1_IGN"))
 (segment (start 45.55 26) (end 45.55 25.3983) (width 0.2) (layer "F.Cu") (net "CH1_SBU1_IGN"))
 (segment (start 46.8819 25.3983) (end 47.0548 25.5712) (width 0.2) (layer "F.Cu") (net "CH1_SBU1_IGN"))
 (segment (start 24.46 32.2004) (end 30.4237 26.2367) (width 0.2) (layer "F.Cu") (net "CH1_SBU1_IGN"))
 (segment (start 55.8522 32.4979) (end 55.467 32.4979) (width 0.2) (layer "F.Cu") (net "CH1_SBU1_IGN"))
 (segment (start 47.0548 26.6094) (end 47.0548 26.1358) (width 0.2) (layer "F.Cu") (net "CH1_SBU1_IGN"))
 (segment (start 47.0548 25.5712) (end 47.0548 26.1358) (width 0.2) (layer "F.Cu") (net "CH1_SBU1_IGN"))
 (segment (start 30.4237 26.2367) (end 39.4634 26.2367) (width 0.2) (layer "F.Cu") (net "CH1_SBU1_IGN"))
 (segment (start 25.73 35.27) (end 24.46 34) (width 0.2) (layer "F.Cu") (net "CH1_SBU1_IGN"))
 (segment (start 39.4634 26.2367) (end 40.2398 27.0131) (width 0.2) (layer "F.Cu") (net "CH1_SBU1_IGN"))
 (segment (start 61.05 27.3001) (end 55.8522 32.4979) (width 0.2) (layer "F.Cu") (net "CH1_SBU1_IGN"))
 (segment (start 55.9898 26.1358) (end 57.1541 27.3001) (width 0.2) (layer "F.Cu") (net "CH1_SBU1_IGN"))
 (segment (start 54.7895 49.1757) (end 54.5669 49.3983) (width 0.2) (layer "F.Cu") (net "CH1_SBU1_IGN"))
 (segment (start 57.1541 27.3001) (end 61.05 27.3001) (width 0.2) (layer "F.Cu") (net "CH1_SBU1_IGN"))
 (segment (start 24.46 34) (end 24.46 32.2004) (width 0.2) (layer "F.Cu") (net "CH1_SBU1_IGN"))
 (segment (start 46.6511 27.0131) (end 47.0548 26.6094) (width 0.2) (layer "F.Cu") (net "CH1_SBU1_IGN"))
 (segment (start 40.2398 27.0131) (end 46.6511 27.0131) (width 0.2) (layer "F.Cu") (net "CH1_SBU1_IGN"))
 (segment (start 45.55 25.3983) (end 46.8819 25.3983) (width 0.2) (layer "F.Cu") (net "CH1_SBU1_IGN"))
 (segment (start 54.5669 49.3983) (end 54.45 49.3983) (width 0.2) (layer "F.Cu") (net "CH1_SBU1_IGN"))
 (segment (start 47.0548 26.1358) (end 55.9898 26.1358) (width 0.2) (layer "F.Cu") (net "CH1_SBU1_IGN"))
 (via (at 54.7895 49.1757) (size 0.6) (drill 0.3) (layers "F.Cu" "B.Cu") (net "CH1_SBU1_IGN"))
 (via (at 55.467 32.4979) (size 0.6) (drill 0.3) (layers "F.Cu" "B.Cu") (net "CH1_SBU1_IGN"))
 (segment (start 54.7895 33.1754) (end 55.467 32.4979) (width 0.2) (layer "B.Cu") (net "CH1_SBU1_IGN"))
 (segment (start 54.7895 49.1757) (end 54.7895 33.1754) (width 0.2) (layer "B.Cu") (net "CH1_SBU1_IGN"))
 (segment (start 59.8163 40.868) (end 60.9483 42) (width 0.2) (layer "F.Cu") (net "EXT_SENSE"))
 (segment (start 46.3911 40.868) (end 59.8163 40.868) (width 0.2) (layer "F.Cu") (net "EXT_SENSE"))
 (segment (start 61.55 42) (end 60.9483 42) (width 0.2) (layer "F.Cu") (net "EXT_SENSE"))
 (via (at 46.3911 40.868) (size 0.6) (drill 0.3) (layers "F.Cu" "B.Cu") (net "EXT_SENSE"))
 (segment (start 31.3623 34) (end 32.0515 34.6892) (width 0.2) (layer "B.Cu") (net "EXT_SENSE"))
 (segment (start 32.0515 39.0609) (end 40.1366 47.146) (width 0.2) (layer "B.Cu") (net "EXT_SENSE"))
 (segment (start 32.0515 34.6892) (end 32.0515 39.0609) (width 0.2) (layer "B.Cu") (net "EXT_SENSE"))
 (segment (start 40.6418 47.146) (end 46.3911 41.3967) (width 0.2) (layer "B.Cu") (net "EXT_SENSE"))
 (segment (start 40.1366 47.146) (end 40.6418 47.146) (width 0.2) (layer "B.Cu") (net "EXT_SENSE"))
 (segment (start 28.9462 32.73) (end 30.2162 34) (width 0.2) (layer "B.Cu") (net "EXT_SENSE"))
 (segment (start 28.27 32.73) (end 28.9462 32.73) (width 0.2) (layer "B.Cu") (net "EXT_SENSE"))
 (segment (start 30.2162 34) (end 31.3623 34) (width 0.2) (layer "B.Cu") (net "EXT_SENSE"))
 (segment (start 46.3911 41.3967) (end 46.3911 40.868) (width 0.2) (layer "B.Cu") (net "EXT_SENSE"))
 (segment (start 49.4697 46.5214) (end 52.9483 50) (width 0.2) (layer "F.Cu") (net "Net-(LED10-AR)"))
 (segment (start 37.05 27) (end 37.7517 27) (width 0.2) (layer "F.Cu") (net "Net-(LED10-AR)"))
 (segment (start 37.7517 27) (end 37.8298 27.0781) (width 0.2) (layer "F.Cu") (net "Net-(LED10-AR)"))
 (segment (start 37.8298 27.0781) (end 37.9568 27.0781) (width 0.2) (layer "F.Cu") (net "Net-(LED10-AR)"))
 (segment (start 53.55 50) (end 52.9483 50) (width 0.2) (layer "F.Cu") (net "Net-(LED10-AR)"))
 (segment (start 40.3947 46.5214) (end 49.4697 46.5214) (width 0.2) (layer "F.Cu") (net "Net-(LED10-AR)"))
 (via (at 40.3947 46.5214) (size 0.6) (drill 0.3) (layers "F.Cu" "B.Cu") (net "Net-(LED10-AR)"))
 (via (at 37.9568 27.0781) (size 0.6) (drill 0.3) (layers "F.Cu" "B.Cu") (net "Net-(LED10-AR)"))
 (segment (start 37.9568 27.0781) (end 37.9568 44.0835) (width 0.2) (layer "B.Cu") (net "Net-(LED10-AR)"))
 (segment (start 37.9568 44.0835) (end 40.3947 46.5214) (width 0.2) (layer "B.Cu") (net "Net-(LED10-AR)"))
 (segment (start 46.65 27.7017) (end 40.3534 27.7017) (width 0.2) (layer "F.Cu") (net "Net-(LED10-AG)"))
 (segment (start 40.3534 27.7017) (end 39.6517 27) (width 0.2) (layer "F.Cu") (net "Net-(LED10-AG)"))
 (segment (start 38.95 27) (end 39.6517 27) (width 0.2) (layer "F.Cu") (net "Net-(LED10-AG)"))
 (segment (start 52.9483 34) (end 46.65 27.7017) (width 0.2) (layer "F.Cu") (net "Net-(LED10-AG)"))
 (segment (start 53.55 34) (end 52.9483 34) (width 0.2) (layer "F.Cu") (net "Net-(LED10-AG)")))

